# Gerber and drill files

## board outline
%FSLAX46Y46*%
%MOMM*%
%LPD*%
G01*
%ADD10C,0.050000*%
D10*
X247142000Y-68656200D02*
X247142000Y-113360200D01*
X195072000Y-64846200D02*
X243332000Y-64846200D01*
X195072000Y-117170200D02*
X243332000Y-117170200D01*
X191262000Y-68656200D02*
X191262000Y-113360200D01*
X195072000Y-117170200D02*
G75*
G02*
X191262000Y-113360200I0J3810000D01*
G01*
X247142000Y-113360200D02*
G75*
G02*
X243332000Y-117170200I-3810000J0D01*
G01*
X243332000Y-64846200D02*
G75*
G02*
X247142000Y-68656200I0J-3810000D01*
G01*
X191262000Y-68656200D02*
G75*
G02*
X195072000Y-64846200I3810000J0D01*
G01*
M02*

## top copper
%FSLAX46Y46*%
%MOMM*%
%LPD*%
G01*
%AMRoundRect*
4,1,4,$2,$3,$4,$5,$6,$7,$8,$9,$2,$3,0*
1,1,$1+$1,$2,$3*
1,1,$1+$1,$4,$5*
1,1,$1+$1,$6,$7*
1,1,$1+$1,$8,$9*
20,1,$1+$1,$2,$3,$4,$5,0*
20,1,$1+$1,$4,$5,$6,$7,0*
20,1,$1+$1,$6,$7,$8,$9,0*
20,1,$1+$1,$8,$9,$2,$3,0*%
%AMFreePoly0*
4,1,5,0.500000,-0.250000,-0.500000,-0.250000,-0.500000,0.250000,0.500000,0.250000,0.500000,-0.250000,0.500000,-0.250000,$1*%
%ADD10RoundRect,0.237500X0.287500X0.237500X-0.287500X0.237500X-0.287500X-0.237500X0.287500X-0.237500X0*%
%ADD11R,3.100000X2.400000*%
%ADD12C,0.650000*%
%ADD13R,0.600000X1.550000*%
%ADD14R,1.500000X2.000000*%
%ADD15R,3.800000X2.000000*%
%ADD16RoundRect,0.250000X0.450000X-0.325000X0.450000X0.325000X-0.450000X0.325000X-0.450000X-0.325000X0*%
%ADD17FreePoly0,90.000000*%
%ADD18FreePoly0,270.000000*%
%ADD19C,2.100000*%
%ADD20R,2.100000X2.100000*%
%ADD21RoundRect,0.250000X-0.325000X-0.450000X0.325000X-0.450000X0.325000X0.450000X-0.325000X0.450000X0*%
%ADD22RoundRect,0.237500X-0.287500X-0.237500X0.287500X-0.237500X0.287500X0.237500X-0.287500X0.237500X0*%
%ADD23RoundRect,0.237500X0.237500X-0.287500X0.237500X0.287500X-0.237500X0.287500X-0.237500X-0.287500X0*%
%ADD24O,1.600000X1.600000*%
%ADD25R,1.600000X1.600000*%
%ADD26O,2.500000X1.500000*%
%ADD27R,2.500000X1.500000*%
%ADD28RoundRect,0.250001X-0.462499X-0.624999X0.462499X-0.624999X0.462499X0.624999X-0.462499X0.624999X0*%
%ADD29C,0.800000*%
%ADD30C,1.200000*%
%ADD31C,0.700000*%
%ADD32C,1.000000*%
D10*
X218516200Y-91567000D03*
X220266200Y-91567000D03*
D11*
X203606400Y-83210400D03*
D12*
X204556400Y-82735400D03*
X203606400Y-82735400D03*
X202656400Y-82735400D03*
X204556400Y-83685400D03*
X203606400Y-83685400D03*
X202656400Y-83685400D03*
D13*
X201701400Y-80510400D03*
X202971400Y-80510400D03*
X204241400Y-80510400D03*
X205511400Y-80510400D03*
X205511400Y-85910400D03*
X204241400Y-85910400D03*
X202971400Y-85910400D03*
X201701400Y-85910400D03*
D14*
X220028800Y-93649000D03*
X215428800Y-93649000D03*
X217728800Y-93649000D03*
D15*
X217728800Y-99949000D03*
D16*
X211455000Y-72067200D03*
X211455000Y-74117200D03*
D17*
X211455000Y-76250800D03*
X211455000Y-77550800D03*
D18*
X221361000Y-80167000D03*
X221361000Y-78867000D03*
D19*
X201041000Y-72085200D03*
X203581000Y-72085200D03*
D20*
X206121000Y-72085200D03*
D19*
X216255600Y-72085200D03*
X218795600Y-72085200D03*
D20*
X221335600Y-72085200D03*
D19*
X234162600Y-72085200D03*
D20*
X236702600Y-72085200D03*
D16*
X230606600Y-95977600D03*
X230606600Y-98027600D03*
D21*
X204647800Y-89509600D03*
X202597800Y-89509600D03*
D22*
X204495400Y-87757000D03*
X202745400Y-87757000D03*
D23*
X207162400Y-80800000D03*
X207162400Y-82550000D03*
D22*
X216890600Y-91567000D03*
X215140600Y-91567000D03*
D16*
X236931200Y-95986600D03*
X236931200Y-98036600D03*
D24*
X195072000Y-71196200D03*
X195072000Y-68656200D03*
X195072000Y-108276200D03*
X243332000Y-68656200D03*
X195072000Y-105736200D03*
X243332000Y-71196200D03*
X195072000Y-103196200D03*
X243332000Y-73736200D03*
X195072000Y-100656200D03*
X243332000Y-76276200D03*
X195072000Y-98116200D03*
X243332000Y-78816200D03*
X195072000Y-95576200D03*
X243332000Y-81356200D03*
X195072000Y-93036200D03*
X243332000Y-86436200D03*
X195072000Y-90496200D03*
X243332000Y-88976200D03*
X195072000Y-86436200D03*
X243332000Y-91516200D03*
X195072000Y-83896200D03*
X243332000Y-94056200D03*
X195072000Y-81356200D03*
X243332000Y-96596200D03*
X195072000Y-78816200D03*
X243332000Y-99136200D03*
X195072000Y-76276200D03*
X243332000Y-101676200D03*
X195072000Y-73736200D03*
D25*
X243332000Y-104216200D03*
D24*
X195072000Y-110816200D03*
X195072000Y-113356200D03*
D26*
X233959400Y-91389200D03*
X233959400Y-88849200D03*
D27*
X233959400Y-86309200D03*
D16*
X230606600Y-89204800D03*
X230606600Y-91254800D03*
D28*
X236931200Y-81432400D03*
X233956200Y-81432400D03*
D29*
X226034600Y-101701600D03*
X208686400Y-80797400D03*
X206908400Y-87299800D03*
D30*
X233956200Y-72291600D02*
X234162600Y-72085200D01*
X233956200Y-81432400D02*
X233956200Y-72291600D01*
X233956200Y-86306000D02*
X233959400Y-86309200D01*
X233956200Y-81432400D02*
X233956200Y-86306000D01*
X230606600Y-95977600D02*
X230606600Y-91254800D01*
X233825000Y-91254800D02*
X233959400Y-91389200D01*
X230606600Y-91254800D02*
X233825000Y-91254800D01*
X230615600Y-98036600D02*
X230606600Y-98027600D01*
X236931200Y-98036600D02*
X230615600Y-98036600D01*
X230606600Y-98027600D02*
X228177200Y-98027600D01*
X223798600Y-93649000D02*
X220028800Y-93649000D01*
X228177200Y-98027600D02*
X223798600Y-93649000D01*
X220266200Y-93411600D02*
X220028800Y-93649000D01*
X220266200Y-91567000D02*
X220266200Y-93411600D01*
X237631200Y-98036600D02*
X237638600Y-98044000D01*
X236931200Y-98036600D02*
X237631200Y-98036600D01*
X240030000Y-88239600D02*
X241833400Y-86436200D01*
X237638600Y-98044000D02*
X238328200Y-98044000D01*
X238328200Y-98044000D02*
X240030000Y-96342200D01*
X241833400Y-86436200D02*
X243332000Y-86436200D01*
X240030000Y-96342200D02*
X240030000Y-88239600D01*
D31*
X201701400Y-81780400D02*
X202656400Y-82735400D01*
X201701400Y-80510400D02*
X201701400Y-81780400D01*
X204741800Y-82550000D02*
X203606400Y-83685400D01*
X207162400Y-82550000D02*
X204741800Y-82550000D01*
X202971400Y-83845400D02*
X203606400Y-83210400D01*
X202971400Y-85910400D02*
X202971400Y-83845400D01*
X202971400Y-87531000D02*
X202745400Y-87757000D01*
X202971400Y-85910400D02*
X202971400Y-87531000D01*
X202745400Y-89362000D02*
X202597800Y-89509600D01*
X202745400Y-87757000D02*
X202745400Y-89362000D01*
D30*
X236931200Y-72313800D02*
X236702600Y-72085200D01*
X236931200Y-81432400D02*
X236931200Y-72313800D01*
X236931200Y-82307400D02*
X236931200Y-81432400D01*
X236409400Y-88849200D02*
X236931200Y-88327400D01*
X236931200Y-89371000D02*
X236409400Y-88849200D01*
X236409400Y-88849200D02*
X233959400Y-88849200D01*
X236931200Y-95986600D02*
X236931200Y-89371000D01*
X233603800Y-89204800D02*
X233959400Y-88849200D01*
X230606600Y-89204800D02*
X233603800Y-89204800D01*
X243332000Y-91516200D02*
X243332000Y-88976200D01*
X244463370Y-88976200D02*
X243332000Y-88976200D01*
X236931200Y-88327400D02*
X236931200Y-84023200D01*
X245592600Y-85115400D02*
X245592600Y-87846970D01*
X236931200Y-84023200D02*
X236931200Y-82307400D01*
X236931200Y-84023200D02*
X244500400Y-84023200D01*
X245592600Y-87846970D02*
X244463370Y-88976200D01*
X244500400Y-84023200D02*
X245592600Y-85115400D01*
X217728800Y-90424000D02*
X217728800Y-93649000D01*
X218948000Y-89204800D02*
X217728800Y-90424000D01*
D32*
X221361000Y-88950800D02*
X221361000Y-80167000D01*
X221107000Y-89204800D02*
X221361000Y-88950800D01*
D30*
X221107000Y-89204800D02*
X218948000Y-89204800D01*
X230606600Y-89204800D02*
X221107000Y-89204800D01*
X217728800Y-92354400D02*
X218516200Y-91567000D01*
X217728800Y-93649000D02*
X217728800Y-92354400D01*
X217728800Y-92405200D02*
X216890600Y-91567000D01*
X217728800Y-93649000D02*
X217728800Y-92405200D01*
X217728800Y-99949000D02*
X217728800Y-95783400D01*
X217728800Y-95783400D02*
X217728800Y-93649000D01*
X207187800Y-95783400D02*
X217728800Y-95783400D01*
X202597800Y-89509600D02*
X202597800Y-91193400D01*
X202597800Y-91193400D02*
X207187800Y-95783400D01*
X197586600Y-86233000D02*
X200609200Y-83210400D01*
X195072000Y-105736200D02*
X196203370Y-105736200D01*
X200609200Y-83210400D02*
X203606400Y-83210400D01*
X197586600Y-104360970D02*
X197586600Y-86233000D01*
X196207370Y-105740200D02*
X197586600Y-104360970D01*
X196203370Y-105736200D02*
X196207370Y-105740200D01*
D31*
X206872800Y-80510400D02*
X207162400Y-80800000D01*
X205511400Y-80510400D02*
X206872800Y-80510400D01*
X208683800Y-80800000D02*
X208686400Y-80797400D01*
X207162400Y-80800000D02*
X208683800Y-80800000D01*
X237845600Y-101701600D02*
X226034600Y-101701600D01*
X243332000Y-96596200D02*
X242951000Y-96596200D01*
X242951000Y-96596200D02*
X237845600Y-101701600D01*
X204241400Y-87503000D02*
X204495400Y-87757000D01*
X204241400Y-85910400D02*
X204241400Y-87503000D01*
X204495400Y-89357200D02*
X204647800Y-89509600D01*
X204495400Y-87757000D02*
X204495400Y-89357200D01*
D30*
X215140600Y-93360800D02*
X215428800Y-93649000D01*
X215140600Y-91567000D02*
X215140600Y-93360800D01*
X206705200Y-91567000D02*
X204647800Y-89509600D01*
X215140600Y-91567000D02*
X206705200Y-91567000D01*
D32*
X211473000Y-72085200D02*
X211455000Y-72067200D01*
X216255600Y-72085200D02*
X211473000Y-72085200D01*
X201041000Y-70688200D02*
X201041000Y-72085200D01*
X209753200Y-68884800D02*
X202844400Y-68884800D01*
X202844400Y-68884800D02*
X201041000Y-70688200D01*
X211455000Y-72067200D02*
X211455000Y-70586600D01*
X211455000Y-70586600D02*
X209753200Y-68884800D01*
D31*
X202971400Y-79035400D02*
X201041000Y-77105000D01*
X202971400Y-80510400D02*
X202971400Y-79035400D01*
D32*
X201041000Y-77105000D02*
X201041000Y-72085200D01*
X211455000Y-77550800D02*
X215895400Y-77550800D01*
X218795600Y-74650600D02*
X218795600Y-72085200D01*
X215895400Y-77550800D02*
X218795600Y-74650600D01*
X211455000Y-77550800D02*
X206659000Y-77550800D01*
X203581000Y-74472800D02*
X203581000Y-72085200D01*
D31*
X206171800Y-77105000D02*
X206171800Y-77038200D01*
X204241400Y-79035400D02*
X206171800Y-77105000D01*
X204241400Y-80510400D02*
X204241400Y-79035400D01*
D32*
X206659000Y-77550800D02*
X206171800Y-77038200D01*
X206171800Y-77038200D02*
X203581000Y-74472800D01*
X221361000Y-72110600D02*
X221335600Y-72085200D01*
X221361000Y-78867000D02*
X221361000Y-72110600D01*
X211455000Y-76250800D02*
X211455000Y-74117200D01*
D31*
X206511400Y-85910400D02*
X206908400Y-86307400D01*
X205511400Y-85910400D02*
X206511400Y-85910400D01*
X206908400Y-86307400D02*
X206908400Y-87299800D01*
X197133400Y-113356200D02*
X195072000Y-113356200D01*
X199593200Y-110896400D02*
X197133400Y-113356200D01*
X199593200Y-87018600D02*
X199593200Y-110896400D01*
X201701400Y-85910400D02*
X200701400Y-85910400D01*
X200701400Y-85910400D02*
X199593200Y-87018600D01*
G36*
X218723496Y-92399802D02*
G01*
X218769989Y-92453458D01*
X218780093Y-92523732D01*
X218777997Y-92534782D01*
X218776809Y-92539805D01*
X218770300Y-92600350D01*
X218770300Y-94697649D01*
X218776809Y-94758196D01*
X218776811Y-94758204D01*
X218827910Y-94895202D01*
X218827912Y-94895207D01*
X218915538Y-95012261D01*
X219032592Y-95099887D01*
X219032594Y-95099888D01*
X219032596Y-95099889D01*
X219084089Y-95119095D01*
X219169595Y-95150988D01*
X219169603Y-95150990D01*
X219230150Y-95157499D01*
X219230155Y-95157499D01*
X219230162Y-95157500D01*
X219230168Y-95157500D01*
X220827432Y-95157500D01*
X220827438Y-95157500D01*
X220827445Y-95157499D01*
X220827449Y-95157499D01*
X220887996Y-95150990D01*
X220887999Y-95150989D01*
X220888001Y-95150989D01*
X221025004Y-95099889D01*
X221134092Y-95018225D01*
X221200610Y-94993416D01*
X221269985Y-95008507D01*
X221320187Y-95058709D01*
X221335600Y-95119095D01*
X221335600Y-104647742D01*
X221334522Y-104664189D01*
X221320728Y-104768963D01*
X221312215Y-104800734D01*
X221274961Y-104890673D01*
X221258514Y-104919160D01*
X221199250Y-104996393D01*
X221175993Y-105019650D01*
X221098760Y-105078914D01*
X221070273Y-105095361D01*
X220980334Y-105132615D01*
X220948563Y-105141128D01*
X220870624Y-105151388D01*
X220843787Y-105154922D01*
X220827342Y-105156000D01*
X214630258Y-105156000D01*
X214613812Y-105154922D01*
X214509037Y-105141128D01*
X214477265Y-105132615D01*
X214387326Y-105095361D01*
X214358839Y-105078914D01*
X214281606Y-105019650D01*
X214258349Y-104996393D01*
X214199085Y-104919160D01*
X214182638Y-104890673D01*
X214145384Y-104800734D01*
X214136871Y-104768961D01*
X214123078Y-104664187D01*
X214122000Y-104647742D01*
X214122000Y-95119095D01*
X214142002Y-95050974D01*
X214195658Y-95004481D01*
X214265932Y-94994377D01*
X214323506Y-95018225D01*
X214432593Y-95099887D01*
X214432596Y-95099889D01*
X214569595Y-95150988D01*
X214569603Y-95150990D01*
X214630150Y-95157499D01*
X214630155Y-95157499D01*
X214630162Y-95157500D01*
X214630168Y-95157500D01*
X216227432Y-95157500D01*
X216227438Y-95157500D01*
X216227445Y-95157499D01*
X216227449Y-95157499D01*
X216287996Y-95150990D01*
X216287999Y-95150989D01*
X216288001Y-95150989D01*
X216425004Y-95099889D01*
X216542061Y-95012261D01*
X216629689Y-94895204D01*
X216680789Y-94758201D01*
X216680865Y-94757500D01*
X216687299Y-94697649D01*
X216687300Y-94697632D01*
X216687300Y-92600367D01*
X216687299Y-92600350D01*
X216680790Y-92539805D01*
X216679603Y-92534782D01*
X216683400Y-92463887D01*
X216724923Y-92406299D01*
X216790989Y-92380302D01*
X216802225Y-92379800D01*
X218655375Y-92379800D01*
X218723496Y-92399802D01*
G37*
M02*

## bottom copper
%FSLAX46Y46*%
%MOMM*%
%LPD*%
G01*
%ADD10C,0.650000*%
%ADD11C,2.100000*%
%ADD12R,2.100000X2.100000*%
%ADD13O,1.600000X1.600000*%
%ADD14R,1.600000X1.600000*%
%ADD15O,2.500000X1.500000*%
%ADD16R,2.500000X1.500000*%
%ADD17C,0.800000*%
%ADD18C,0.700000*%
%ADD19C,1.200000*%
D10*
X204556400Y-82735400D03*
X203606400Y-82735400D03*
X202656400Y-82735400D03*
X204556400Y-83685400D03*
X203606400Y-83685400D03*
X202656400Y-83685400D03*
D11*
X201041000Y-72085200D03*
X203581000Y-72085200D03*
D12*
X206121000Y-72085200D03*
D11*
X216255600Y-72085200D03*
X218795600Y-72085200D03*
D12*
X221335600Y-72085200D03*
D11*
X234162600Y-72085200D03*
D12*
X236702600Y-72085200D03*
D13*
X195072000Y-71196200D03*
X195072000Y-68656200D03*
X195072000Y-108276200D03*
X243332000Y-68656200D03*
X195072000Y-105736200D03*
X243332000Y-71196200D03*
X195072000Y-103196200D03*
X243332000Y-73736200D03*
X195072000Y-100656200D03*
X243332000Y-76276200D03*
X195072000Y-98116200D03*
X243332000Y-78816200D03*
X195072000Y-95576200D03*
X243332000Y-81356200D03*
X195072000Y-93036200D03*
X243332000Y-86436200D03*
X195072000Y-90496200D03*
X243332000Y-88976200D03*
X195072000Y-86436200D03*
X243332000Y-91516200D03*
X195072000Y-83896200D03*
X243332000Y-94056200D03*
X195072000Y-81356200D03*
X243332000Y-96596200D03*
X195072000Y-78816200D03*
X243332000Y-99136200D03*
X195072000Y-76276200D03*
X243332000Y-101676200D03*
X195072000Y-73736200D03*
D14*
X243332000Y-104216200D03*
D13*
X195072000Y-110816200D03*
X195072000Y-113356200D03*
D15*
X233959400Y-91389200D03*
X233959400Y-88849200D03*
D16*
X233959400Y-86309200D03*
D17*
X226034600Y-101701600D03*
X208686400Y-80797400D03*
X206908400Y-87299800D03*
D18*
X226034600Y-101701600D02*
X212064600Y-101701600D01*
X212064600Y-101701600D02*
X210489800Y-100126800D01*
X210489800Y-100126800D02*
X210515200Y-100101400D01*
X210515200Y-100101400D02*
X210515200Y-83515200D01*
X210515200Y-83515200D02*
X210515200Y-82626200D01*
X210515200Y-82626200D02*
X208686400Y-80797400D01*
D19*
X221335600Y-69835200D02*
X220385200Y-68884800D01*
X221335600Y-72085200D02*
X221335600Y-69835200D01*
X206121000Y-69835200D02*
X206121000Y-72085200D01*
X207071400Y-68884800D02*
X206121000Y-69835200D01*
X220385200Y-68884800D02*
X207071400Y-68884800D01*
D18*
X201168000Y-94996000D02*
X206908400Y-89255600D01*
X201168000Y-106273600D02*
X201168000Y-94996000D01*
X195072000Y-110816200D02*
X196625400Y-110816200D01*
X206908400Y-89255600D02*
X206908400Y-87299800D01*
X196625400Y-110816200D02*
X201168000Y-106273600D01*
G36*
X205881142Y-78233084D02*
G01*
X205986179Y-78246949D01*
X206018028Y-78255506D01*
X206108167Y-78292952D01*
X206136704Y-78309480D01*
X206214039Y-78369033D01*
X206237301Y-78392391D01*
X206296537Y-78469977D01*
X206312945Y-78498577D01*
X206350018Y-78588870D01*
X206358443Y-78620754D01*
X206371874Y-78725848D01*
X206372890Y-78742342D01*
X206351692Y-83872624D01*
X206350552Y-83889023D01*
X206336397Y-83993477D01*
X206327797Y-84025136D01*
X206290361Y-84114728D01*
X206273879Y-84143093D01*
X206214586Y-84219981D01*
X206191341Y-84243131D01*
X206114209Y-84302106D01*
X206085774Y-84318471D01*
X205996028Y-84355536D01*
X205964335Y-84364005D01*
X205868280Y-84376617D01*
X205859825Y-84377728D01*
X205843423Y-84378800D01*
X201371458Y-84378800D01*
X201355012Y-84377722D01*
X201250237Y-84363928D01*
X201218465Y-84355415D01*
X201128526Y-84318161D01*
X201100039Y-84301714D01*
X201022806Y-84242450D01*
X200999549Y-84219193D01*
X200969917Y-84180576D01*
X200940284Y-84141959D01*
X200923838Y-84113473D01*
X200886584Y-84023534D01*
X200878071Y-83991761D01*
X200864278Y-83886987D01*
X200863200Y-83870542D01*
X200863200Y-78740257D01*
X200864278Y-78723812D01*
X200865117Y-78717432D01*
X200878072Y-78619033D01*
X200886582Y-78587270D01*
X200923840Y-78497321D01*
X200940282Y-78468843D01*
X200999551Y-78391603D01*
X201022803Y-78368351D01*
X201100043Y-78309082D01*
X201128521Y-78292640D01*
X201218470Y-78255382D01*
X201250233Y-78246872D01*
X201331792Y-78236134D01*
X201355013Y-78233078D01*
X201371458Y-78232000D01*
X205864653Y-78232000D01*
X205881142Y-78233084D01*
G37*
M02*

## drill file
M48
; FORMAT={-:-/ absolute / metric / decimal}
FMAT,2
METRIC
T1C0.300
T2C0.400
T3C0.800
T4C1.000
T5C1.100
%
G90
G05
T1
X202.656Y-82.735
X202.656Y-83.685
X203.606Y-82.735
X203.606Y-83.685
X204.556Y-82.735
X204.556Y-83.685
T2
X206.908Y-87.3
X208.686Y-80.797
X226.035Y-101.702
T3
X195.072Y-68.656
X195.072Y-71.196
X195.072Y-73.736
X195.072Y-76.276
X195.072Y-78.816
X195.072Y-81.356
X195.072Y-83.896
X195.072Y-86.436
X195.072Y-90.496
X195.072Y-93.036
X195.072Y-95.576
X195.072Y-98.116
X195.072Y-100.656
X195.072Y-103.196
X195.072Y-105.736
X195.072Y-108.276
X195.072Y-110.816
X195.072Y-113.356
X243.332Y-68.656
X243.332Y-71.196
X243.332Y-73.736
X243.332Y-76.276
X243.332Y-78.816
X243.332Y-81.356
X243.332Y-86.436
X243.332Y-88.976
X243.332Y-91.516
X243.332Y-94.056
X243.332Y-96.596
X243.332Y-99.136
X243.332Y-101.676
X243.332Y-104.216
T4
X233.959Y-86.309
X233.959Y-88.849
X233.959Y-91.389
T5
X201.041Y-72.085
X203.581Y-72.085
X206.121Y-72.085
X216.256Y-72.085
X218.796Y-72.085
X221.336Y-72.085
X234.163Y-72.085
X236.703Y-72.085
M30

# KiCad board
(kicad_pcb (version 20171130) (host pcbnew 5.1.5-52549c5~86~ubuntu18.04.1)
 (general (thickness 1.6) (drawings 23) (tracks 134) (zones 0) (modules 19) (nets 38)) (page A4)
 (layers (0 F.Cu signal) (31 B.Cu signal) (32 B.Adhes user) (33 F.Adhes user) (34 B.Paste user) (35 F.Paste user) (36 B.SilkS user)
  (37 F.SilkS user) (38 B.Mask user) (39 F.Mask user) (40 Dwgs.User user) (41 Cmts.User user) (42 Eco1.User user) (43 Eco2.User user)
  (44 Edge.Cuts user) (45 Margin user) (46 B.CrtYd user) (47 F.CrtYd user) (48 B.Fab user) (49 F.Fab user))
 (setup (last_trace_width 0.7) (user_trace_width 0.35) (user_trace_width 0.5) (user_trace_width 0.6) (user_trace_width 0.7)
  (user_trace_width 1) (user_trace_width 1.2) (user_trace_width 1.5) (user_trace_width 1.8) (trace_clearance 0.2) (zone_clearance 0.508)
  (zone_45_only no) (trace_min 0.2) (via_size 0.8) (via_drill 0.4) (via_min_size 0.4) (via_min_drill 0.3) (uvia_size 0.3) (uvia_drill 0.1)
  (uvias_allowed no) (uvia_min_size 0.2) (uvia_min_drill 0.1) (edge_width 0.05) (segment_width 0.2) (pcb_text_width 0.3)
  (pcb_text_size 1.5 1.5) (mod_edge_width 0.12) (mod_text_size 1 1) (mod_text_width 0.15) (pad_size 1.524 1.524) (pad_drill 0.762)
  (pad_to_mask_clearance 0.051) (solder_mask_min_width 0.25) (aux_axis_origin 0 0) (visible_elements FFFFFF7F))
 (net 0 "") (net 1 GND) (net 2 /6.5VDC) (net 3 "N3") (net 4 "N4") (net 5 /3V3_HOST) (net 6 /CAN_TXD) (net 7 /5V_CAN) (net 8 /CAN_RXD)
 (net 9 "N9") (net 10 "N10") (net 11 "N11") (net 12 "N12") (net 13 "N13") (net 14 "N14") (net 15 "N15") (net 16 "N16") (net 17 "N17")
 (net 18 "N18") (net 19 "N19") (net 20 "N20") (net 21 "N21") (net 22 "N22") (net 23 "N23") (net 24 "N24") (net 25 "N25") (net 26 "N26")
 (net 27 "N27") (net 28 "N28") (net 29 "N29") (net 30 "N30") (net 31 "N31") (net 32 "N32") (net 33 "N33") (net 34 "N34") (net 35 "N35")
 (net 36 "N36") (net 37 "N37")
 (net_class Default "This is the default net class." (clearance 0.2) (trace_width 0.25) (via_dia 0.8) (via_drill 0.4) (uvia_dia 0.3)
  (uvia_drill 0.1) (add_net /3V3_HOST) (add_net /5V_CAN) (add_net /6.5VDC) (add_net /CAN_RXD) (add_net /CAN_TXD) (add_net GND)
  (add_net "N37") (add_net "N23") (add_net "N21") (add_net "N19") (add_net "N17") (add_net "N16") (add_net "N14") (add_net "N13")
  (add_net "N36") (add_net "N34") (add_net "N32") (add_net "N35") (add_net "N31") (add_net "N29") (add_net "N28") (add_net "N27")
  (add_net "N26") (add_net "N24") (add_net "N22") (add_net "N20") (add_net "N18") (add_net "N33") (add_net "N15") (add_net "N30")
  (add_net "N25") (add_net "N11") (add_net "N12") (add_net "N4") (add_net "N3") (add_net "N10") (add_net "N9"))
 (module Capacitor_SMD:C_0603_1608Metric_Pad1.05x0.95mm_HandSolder (layer F.Cu) (at 219.3912 91.567 180)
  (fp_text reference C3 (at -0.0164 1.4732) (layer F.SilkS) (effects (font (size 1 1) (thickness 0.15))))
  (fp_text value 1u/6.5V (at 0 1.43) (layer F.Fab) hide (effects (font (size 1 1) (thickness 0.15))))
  (pad 2 smd roundrect (at 0.875 0 180) (size 1.05 0.95) (layers F.Cu F.Paste F.Mask) (roundrect_rratio 0.25) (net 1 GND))
  (pad 1 smd roundrect (at -0.875 0 180) (size 1.05 0.95) (layers F.Cu F.Paste F.Mask) (roundrect_rratio 0.25) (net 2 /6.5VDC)))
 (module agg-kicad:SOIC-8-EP (layer F.Cu) (at 203.6064 83.2104 90)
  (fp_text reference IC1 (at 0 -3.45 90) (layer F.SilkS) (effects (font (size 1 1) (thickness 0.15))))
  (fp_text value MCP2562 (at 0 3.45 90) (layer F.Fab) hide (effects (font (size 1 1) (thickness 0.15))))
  (pad EP smd rect (at 0 0 90) (size 2.4 3.1) (layers F.Cu F.Paste F.Mask) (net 1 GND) (solder_mask_margin 0.001)
   (solder_paste_margin 0.001))
  (pad EP thru_hole circle (at 0.475 0.95 90) (size 0.65 0.65) (drill 0.3) (layers *.Cu) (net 1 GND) (zone_connect 2))
  (pad EP thru_hole circle (at 0.475 0 90) (size 0.65 0.65) (drill 0.3) (layers *.Cu) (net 1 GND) (zone_connect 2))
  (pad EP thru_hole circle (at 0.475 -0.95 90) (size 0.65 0.65) (drill 0.3) (layers *.Cu) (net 1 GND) (zone_connect 2))
  (pad EP thru_hole circle (at -0.475 0.95 90) (size 0.65 0.65) (drill 0.3) (layers *.Cu) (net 1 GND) (zone_connect 2))
  (pad EP thru_hole circle (at -0.475 0 90) (size 0.65 0.65) (drill 0.3) (layers *.Cu) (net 1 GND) (zone_connect 2))
  (pad EP thru_hole circle (at -0.475 -0.95 90) (size 0.65 0.65) (drill 0.3) (layers *.Cu) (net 1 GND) (zone_connect 2))
  (pad 8 smd rect (at 2.7 -1.905 90) (size 1.55 0.6) (layers F.Cu F.Paste F.Mask) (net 1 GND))
  (pad 7 smd rect (at 2.7 -0.635 90) (size 1.55 0.6) (layers F.Cu F.Paste F.Mask) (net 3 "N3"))
  (pad 6 smd rect (at 2.7 0.635 90) (size 1.55 0.6) (layers F.Cu F.Paste F.Mask) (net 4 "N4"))
  (pad 5 smd rect (at 2.7 1.905 90) (size 1.55 0.6) (layers F.Cu F.Paste F.Mask) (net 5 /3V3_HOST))
  (pad 4 smd rect (at -2.7 1.905 90) (size 1.55 0.6) (layers F.Cu F.Paste F.Mask) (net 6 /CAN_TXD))
  (pad 3 smd rect (at -2.7 0.635 90) (size 1.55 0.6) (layers F.Cu F.Paste F.Mask) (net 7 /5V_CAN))
  (pad 2 smd rect (at -2.7 -0.635 90) (size 1.55 0.6) (layers F.Cu F.Paste F.Mask) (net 1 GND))
  (pad 1 smd rect (at -2.7 -1.905 90) (size 1.55 0.6) (layers F.Cu F.Paste F.Mask) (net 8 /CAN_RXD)))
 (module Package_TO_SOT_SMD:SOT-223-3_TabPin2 (layer F.Cu) (at 217.7288 96.799 270)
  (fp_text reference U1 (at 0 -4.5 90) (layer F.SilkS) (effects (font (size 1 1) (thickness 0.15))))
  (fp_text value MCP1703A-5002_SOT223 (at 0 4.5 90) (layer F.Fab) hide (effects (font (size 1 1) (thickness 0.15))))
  (pad 1 smd rect (at -3.15 -2.3 270) (size 2 1.5) (layers F.Cu F.Paste F.Mask) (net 2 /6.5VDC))
  (pad 3 smd rect (at -3.15 2.3 270) (size 2 1.5) (layers F.Cu F.Paste F.Mask) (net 7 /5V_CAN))
  (pad 2 smd rect (at -3.15 0 270) (size 2 1.5) (layers F.Cu F.Paste F.Mask) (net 1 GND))
  (pad 2 smd rect (at 3.15 0 270) (size 2 3.8) (layers F.Cu F.Paste F.Mask) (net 1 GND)))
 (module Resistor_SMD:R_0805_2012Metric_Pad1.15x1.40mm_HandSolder (layer F.Cu) (at 211.455 73.0922 90)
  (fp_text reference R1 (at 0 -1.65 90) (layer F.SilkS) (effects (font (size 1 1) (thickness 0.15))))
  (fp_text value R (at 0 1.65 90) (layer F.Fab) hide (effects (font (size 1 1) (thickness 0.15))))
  (pad 2 smd roundrect (at 1.025 0 90) (size 1.15 1.4) (layers F.Cu F.Paste F.Mask) (roundrect_rratio 0.217391) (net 3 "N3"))
  (pad 1 smd roundrect (at -1.025 0 90) (size 1.15 1.4) (layers F.Cu F.Paste F.Mask) (roundrect_rratio 0.217391) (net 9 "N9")))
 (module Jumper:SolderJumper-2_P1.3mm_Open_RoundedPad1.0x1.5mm (layer F.Cu) (at 211.455 76.9008 90)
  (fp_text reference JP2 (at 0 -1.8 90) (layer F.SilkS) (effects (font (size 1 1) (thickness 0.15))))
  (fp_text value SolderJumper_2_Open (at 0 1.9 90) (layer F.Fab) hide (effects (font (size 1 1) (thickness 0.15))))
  (pad 2 smd custom (at 0.65 0 90) (size 1 0.5) (layers F.Cu F.Mask) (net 9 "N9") (zone_connect 2)
   (options (clearance outline) (anchor rect)) (primitives))
  (pad 1 smd custom (at -0.65 0 90) (size 1 0.5) (layers F.Cu F.Mask) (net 4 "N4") (zone_connect 2)
   (options (clearance outline) (anchor rect)) (primitives)))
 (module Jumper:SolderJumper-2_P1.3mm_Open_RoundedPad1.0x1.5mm (layer F.Cu) (at 221.361 79.517 270)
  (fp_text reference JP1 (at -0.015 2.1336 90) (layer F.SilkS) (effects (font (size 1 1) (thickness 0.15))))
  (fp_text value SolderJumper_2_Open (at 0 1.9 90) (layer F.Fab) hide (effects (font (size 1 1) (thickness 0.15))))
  (pad 2 smd custom (at 0.65 0 270) (size 1 0.5) (layers F.Cu F.Mask) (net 1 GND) (zone_connect 2)
   (options (clearance outline) (anchor rect)) (primitives))
  (pad 1 smd custom (at -0.65 0 270) (size 1 0.5) (layers F.Cu F.Mask) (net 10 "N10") (zone_connect 2)
   (options (clearance outline) (anchor rect)) (primitives)))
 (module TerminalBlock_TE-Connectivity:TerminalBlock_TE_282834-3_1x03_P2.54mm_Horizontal (layer F.Cu) (at 206.121 72.0852 180)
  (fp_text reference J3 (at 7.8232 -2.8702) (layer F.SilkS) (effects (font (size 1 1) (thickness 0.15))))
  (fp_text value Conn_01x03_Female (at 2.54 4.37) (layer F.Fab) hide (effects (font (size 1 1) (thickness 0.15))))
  (pad 3 thru_hole circle (at 5.08 0 180) (size 2.1 2.1) (drill 1.1) (layers *.Cu *.Mask) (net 3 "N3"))
  (pad 2 thru_hole circle (at 2.54 0 180) (size 2.1 2.1) (drill 1.1) (layers *.Cu *.Mask) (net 4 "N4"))
  (pad 1 thru_hole rect (at 0 0 180) (size 2.1 2.1) (drill 1.1) (layers *.Cu *.Mask) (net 10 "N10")))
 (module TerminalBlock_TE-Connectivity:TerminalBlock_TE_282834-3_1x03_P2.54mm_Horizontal (layer F.Cu) (at 221.3356 72.0852 180)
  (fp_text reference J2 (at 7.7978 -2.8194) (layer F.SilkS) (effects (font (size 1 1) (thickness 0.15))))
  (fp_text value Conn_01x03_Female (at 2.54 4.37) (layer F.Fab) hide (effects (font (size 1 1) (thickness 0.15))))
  (pad 3 thru_hole circle (at 5.08 0 180) (size 2.1 2.1) (drill 1.1) (layers *.Cu *.Mask) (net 3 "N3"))
  (pad 2 thru_hole circle (at 2.54 0 180) (size 2.1 2.1) (drill 1.1) (layers *.Cu *.Mask) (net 4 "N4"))
  (pad 1 thru_hole rect (at 0 0 180) (size 2.1 2.1) (drill 1.1) (layers *.Cu *.Mask) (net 10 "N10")))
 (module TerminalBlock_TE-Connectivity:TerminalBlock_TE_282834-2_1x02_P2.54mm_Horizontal (layer F.Cu) (at 236.7026 72.0852 180)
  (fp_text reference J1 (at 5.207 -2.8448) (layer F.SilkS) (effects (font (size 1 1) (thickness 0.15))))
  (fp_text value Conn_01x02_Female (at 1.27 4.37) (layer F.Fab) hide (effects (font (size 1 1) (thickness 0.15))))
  (pad 2 thru_hole circle (at 2.54 0 180) (size 2.1 2.1) (drill 1.1) (layers *.Cu *.Mask) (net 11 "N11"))
  (pad 1 thru_hole rect (at 0 0 180) (size 2.1 2.1) (drill 1.1) (layers *.Cu *.Mask) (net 1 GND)))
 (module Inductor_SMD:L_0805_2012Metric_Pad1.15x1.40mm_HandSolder (layer F.Cu) (at 230.6066 97.0026 90)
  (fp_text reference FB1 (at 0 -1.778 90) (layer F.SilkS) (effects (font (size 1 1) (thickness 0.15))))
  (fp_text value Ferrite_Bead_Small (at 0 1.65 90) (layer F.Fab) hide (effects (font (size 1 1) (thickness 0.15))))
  (pad 2 smd roundrect (at 1.025 0 90) (size 1.15 1.4) (layers F.Cu F.Paste F.Mask) (roundrect_rratio 0.217391) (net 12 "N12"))
  (pad 1 smd roundrect (at -1.025 0 90) (size 1.15 1.4) (layers F.Cu F.Paste F.Mask) (roundrect_rratio 0.217391) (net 2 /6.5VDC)))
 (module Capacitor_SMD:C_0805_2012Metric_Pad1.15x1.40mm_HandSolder (layer F.Cu) (at 203.6228 89.5096)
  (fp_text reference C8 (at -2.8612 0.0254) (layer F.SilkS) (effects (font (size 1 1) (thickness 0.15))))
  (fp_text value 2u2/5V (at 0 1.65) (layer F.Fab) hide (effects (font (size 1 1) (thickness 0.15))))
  (pad 2 smd roundrect (at 1.025 0) (size 1.15 1.4) (layers F.Cu F.Paste F.Mask) (roundrect_rratio 0.217391) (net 7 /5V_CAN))
  (pad 1 smd roundrect (at -1.025 0) (size 1.15 1.4) (layers F.Cu F.Paste F.Mask) (roundrect_rratio 0.217391) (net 1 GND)))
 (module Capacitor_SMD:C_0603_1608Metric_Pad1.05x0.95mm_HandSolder (layer F.Cu) (at 203.6204 87.757)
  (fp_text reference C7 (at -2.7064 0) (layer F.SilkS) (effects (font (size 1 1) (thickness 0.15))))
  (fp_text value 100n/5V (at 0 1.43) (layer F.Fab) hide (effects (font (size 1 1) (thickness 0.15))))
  (pad 2 smd roundrect (at 0.875 0) (size 1.05 0.95) (layers F.Cu F.Paste F.Mask) (roundrect_rratio 0.25) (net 7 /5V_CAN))
  (pad 1 smd roundrect (at -0.875 0) (size 1.05 0.95) (layers F.Cu F.Paste F.Mask) (roundrect_rratio 0.25) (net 1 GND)))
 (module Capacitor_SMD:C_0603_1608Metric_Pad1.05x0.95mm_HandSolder (layer F.Cu) (at 207.1624 81.675 90)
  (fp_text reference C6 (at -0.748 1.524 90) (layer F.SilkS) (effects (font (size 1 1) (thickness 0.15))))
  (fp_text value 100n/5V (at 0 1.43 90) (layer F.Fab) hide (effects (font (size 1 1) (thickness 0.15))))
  (pad 2 smd roundrect (at 0.875 0 90) (size 1.05 0.95) (layers F.Cu F.Paste F.Mask) (roundrect_rratio 0.25) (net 5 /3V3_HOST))
  (pad 1 smd roundrect (at -0.875 0 90) (size 1.05 0.95) (layers F.Cu F.Paste F.Mask) (roundrect_rratio 0.25) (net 1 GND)))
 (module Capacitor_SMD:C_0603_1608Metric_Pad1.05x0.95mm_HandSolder (layer F.Cu) (at 216.0156 91.567)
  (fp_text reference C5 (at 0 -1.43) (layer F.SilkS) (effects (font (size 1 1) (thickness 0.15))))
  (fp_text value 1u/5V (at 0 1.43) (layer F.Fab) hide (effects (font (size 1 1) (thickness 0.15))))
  (pad 2 smd roundrect (at 0.875 0) (size 1.05 0.95) (layers F.Cu F.Paste F.Mask) (roundrect_rratio 0.25) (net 1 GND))
  (pad 1 smd roundrect (at -0.875 0) (size 1.05 0.95) (layers F.Cu F.Paste F.Mask) (roundrect_rratio 0.25) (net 7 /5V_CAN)))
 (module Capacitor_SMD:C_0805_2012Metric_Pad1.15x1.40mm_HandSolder (layer F.Cu) (at 236.9312 97.0116 90)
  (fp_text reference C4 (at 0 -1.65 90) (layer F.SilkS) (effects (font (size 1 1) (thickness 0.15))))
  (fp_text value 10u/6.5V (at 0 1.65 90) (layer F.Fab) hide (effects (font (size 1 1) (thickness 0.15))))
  (pad 2 smd roundrect (at 1.025 0 90) (size 1.15 1.4) (layers F.Cu F.Paste F.Mask) (roundrect_rratio 0.217391) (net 1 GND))
  (pad 1 smd roundrect (at -1.025 0 90) (size 1.15 1.4) (layers F.Cu F.Paste F.Mask) (roundrect_rratio 0.217391) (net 2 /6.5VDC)))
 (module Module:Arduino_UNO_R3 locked (layer B.Cu) (at 243.332 104.2162 90)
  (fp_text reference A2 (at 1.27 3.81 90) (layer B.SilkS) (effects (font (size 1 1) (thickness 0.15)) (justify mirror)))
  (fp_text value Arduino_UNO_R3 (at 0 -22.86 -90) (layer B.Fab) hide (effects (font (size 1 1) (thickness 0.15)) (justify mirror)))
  (pad 16 thru_hole oval (at 33.02 -48.26) (size 1.6 1.6) (drill 0.8) (layers *.Cu *.Mask) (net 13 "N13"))
  (pad 15 thru_hole oval (at 35.56 -48.26) (size 1.6 1.6) (drill 0.8) (layers *.Cu *.Mask) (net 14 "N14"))
  (pad 30 thru_hole oval (at -4.06 -48.26) (size 1.6 1.6) (drill 0.8) (layers *.Cu *.Mask) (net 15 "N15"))
  (pad 14 thru_hole oval (at 35.56 0) (size 1.6 1.6) (drill 0.8) (layers *.Cu *.Mask) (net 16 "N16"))
  (pad 29 thru_hole oval (at -1.52 -48.26) (size 1.6 1.6) (drill 0.8) (layers *.Cu *.Mask) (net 1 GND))
  (pad 13 thru_hole oval (at 33.02 0) (size 1.6 1.6) (drill 0.8) (layers *.Cu *.Mask) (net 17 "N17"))
  (pad 28 thru_hole oval (at 1.02 -48.26) (size 1.6 1.6) (drill 0.8) (layers *.Cu *.Mask) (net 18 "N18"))
  (pad 12 thru_hole oval (at 30.48 0) (size 1.6 1.6) (drill 0.8) (layers *.Cu *.Mask) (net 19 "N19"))
  (pad 27 thru_hole oval (at 3.56 -48.26) (size 1.6 1.6) (drill 0.8) (layers *.Cu *.Mask) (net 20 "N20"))
  (pad 11 thru_hole oval (at 27.94 0) (size 1.6 1.6) (drill 0.8) (layers *.Cu *.Mask) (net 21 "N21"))
  (pad 26 thru_hole oval (at 6.1 -48.26) (size 1.6 1.6) (drill 0.8) (layers *.Cu *.Mask) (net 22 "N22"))
  (pad 10 thru_hole oval (at 25.4 0) (size 1.6 1.6) (drill 0.8) (layers *.Cu *.Mask) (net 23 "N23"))
  (pad 25 thru_hole oval (at 8.64 -48.26) (size 1.6 1.6) (drill 0.8) (layers *.Cu *.Mask) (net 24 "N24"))
  (pad 9 thru_hole oval (at 22.86 0) (size 1.6 1.6) (drill 0.8) (layers *.Cu *.Mask) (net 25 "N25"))
  (pad 24 thru_hole oval (at 11.18 -48.26) (size 1.6 1.6) (drill 0.8) (layers *.Cu *.Mask) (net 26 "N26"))
  (pad 8 thru_hole oval (at 17.78 0) (size 1.6 1.6) (drill 0.8) (layers *.Cu *.Mask) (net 2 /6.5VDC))
  (pad 23 thru_hole oval (at 13.72 -48.26) (size 1.6 1.6) (drill 0.8) (layers *.Cu *.Mask) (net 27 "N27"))
  (pad 7 thru_hole oval (at 15.24 0) (size 1.6 1.6) (drill 0.8) (layers *.Cu *.Mask) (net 1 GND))
  (pad 22 thru_hole oval (at 17.78 -48.26) (size 1.6 1.6) (drill 0.8) (layers *.Cu *.Mask) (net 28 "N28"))
  (pad 6 thru_hole oval (at 12.7 0) (size 1.6 1.6) (drill 0.8) (layers *.Cu *.Mask) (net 1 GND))
  (pad 21 thru_hole oval (at 20.32 -48.26) (size 1.6 1.6) (drill 0.8) (layers *.Cu *.Mask) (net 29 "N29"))
  (pad 5 thru_hole oval (at 10.16 0) (size 1.6 1.6) (drill 0.8) (layers *.Cu *.Mask) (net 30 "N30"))
  (pad 20 thru_hole oval (at 22.86 -48.26) (size 1.6 1.6) (drill 0.8) (layers *.Cu *.Mask) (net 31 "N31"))
  (pad 4 thru_hole oval (at 7.62 0) (size 1.6 1.6) (drill 0.8) (layers *.Cu *.Mask) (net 5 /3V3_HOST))
  (pad 19 thru_hole oval (at 25.4 -48.26) (size 1.6 1.6) (drill 0.8) (layers *.Cu *.Mask) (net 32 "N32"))
  (pad 3 thru_hole oval (at 5.08 0) (size 1.6 1.6) (drill 0.8) (layers *.Cu *.Mask) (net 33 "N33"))
  (pad 18 thru_hole oval (at 27.94 -48.26) (size 1.6 1.6) (drill 0.8) (layers *.Cu *.Mask) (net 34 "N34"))
  (pad 2 thru_hole oval (at 2.54 0) (size 1.6 1.6) (drill 0.8) (layers *.Cu *.Mask) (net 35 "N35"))
  (pad 17 thru_hole oval (at 30.48 -48.26) (size 1.6 1.6) (drill 0.8) (layers *.Cu *.Mask) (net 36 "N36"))
  (pad 1 thru_hole rect (at 0 0) (size 1.6 1.6) (drill 0.8) (layers *.Cu *.Mask) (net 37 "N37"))
  (pad 31 thru_hole oval (at -6.6 -48.26) (size 1.6 1.6) (drill 0.8) (layers *.Cu *.Mask) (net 6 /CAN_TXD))
  (pad 32 thru_hole oval (at -9.14 -48.26) (size 1.6 1.6) (drill 0.8) (layers *.Cu *.Mask) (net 8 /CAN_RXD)))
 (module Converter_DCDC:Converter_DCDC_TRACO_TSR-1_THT (layer F.Cu) (at 233.9594 86.3092 270)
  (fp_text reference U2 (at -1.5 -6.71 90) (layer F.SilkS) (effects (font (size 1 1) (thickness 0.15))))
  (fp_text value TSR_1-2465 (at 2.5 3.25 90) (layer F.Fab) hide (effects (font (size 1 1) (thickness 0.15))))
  (pad 3 thru_hole oval (at 5.08 0 270) (size 1.5 2.5) (drill 1) (layers *.Cu *.Mask) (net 12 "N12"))
  (pad 2 thru_hole oval (at 2.54 0 270) (size 1.5 2.5) (drill 1) (layers *.Cu *.Mask) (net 1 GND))
  (pad 1 thru_hole rect (at 0 0 270) (size 1.5 2.5) (drill 1) (layers *.Cu *.Mask) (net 11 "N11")))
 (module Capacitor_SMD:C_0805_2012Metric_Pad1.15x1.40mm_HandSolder (layer F.Cu) (at 230.6066 90.2298 90)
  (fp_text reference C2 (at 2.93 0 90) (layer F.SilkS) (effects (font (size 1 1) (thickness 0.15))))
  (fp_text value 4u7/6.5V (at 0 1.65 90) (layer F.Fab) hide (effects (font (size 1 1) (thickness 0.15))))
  (pad 2 smd roundrect (at 1.025 0 90) (size 1.15 1.4) (layers F.Cu F.Paste F.Mask) (roundrect_rratio 0.217391) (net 1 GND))
  (pad 1 smd roundrect (at -1.025 0 90) (size 1.15 1.4) (layers F.Cu F.Paste F.Mask) (roundrect_rratio 0.217391) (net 12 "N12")))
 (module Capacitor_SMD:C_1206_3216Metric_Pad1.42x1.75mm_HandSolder (layer F.Cu) (at 235.4437 81.4324)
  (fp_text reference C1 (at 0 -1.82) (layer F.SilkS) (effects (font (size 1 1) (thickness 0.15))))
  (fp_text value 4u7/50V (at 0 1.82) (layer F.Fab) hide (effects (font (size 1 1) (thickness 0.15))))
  (pad 2 smd roundrect (at 1.4875 0) (size 1.425 1.75) (layers F.Cu F.Paste F.Mask) (roundrect_rratio 0.175439) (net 1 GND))
  (pad 1 smd roundrect (at -1.4875 0) (size 1.425 1.75) (layers F.Cu F.Paste F.Mask) (roundrect_rratio 0.175439) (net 11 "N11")))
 (gr_line (start 247.142 68.6562) (end 247.142 113.3602) (layer Edge.Cuts) (width 0.05))
 (gr_line (start 195.072 64.8462) (end 243.332 64.8462) (layer Edge.Cuts) (width 0.05))
 (gr_line (start 195.072 117.1702) (end 243.332 117.1702) (layer Edge.Cuts) (width 0.05))
 (gr_line (start 191.262 68.6562) (end 191.262 113.3602) (layer Edge.Cuts) (width 0.05))
 (gr_arc (start 195.072 113.3602) (end 191.262 113.3602) (angle -90) (layer Edge.Cuts) (width 0.05))
 (gr_arc (start 243.332 113.3602) (end 243.332 117.1702) (angle -90) (layer Edge.Cuts) (width 0.05))
 (gr_arc (start 243.332 68.6562) (end 247.142 68.6562) (angle -90) (layer Edge.Cuts) (width 0.05))
 (gr_arc (start 195.072 68.6562) (end 195.072 64.8462) (angle -90) (layer Edge.Cuts) (width 0.05))
 (segment (start 233.9562 72.2916) (end 234.1626 72.0852) (width 1.2) (layer F.Cu) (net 11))
 (segment (start 233.9562 81.4324) (end 233.9562 72.2916) (width 1.2) (layer F.Cu) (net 11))
 (segment (start 233.9562 86.306) (end 233.9594 86.3092) (width 1.2) (layer F.Cu) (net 11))
 (segment (start 233.9562 81.4324) (end 233.9562 86.306) (width 1.2) (layer F.Cu) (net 11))
 (segment (start 230.6066 95.9776) (end 230.6066 91.2548) (width 1.2) (layer F.Cu) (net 12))
 (segment (start 233.825 91.2548) (end 233.9594 91.3892) (width 1.2) (layer F.Cu) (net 12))
 (segment (start 230.6066 91.2548) (end 233.825 91.2548) (width 1.2) (layer F.Cu) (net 12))
 (segment (start 230.6156 98.0366) (end 230.6066 98.0276) (width 1.2) (layer F.Cu) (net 2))
 (segment (start 236.9312 98.0366) (end 230.6156 98.0366) (width 1.2) (layer F.Cu) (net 2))
 (segment (start 230.6066 98.0276) (end 228.1772 98.0276) (width 1.2) (layer F.Cu) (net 2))
 (segment (start 223.7986 93.649) (end 220.0288 93.649) (width 1.2) (layer F.Cu) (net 2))
 (segment (start 228.1772 98.0276) (end 223.7986 93.649) (width 1.2) (layer F.Cu) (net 2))
 (segment (start 220.2662 93.4116) (end 220.0288 93.649) (width 1.2) (layer F.Cu) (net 2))
 (segment (start 220.2662 91.567) (end 220.2662 93.4116) (width 1.2) (layer F.Cu) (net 2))
 (segment (start 237.6312 98.0366) (end 237.6386 98.044) (width 1.2) (layer F.Cu) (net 2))
 (segment (start 236.9312 98.0366) (end 237.6312 98.0366) (width 1.2) (layer F.Cu) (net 2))
 (segment (start 240.03 88.2396) (end 241.8334 86.4362) (width 1.2) (layer F.Cu) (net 2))
 (segment (start 237.6386 98.044) (end 238.3282 98.044) (width 1.2) (layer F.Cu) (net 2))
 (segment (start 238.3282 98.044) (end 240.03 96.3422) (width 1.2) (layer F.Cu) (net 2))
 (segment (start 241.8334 86.4362) (end 243.332 86.4362) (width 1.2) (layer F.Cu) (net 2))
 (segment (start 240.03 96.3422) (end 240.03 88.2396) (width 1.2) (layer F.Cu) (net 2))
 (segment (start 201.7014 81.7804) (end 202.6564 82.7354) (width 0.7) (layer F.Cu) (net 1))
 (segment (start 201.7014 80.5104) (end 201.7014 81.7804) (width 0.7) (layer F.Cu) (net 1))
 (segment (start 204.7418 82.55) (end 203.6064 83.6854) (width 0.7) (layer F.Cu) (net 1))
 (segment (start 207.1624 82.55) (end 204.7418 82.55) (width 0.7) (layer F.Cu) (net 1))
 (segment (start 202.9714 83.8454) (end 203.6064 83.2104) (width 0.7) (layer F.Cu) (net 1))
 (segment (start 202.9714 85.9104) (end 202.9714 83.8454) (width 0.7) (layer F.Cu) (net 1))
 (segment (start 202.9714 87.531) (end 202.7454 87.757) (width 0.7) (layer F.Cu) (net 1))
 (segment (start 202.9714 85.9104) (end 202.9714 87.531) (width 0.7) (layer F.Cu) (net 1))
 (segment (start 202.7454 89.362) (end 202.5978 89.5096) (width 0.7) (layer F.Cu) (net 1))
 (segment (start 202.7454 87.757) (end 202.7454 89.362) (width 0.7) (layer F.Cu) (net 1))
 (segment (start 236.9312 72.3138) (end 236.7026 72.0852) (width 1.2) (layer F.Cu) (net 1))
 (segment (start 236.9312 81.4324) (end 236.9312 72.3138) (width 1.2) (layer F.Cu) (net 1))
 (segment (start 236.9312 82.3074) (end 236.9312 81.4324) (width 1.2) (layer F.Cu) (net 1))
 (segment (start 236.4094 88.8492) (end 236.9312 88.3274) (width 1.2) (layer F.Cu) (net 1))
 (segment (start 236.9312 89.371) (end 236.4094 88.8492) (width 1.2) (layer F.Cu) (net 1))
 (segment (start 236.4094 88.8492) (end 233.9594 88.8492) (width 1.2) (layer F.Cu) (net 1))
 (segment (start 236.9312 95.9866) (end 236.9312 89.371) (width 1.2) (layer F.Cu) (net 1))
 (segment (start 233.6038 89.2048) (end 233.9594 88.8492) (width 1.2) (layer F.Cu) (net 1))
 (segment (start 230.6066 89.2048) (end 233.6038 89.2048) (width 1.2) (layer F.Cu) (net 1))
 (segment (start 243.332 91.5162) (end 243.332 88.9762) (width 1.2) (layer F.Cu) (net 1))
 (segment (start 244.46337 88.9762) (end 243.332 88.9762) (width 1.2) (layer F.Cu) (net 1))
 (segment (start 236.9312 88.3274) (end 236.9312 84.0232) (width 1.2) (layer F.Cu) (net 1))
 (segment (start 245.5926 85.1154) (end 245.5926 87.84697) (width 1.2) (layer F.Cu) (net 1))
 (segment (start 236.9312 84.0232) (end 236.9312 82.3074) (width 1.2) (layer F.Cu) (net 1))
 (segment (start 236.9312 84.0232) (end 244.5004 84.0232) (width 1.2) (layer F.Cu) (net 1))
 (segment (start 245.5926 87.84697) (end 244.46337 88.9762) (width 1.2) (layer F.Cu) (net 1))
 (segment (start 244.5004 84.0232) (end 245.5926 85.1154) (width 1.2) (layer F.Cu) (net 1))
 (segment (start 217.7288 90.424) (end 217.7288 93.649) (width 1.2) (layer F.Cu) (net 1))
 (segment (start 218.948 89.2048) (end 217.7288 90.424) (width 1.2) (layer F.Cu) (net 1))
 (segment (start 221.361 88.9508) (end 221.361 80.167) (width 1) (layer F.Cu) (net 1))
 (segment (start 221.107 89.2048) (end 221.361 88.9508) (width 1) (layer F.Cu) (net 1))
 (segment (start 221.107 89.2048) (end 218.948 89.2048) (width 1.2) (layer F.Cu) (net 1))
 (segment (start 230.6066 89.2048) (end 221.107 89.2048) (width 1.2) (layer F.Cu) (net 1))
 (segment (start 217.7288 92.3544) (end 218.5162 91.567) (width 1.2) (layer F.Cu) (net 1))
 (segment (start 217.7288 93.649) (end 217.7288 92.3544) (width 1.2) (layer F.Cu) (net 1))
 (segment (start 217.7288 92.4052) (end 216.8906 91.567) (width 1.2) (layer F.Cu) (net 1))
 (segment (start 217.7288 93.649) (end 217.7288 92.4052) (width 1.2) (layer F.Cu) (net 1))
 (segment (start 217.7288 99.949) (end 217.7288 95.7834) (width 1.2) (layer F.Cu) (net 1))
 (segment (start 217.7288 95.7834) (end 217.7288 93.649) (width 1.2) (layer F.Cu) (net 1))
 (segment (start 207.1878 95.7834) (end 217.7288 95.7834) (width 1.2) (layer F.Cu) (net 1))
 (segment (start 202.5978 89.5096) (end 202.5978 91.1934) (width 1.2) (layer F.Cu) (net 1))
 (segment (start 202.5978 91.1934) (end 207.1878 95.7834) (width 1.2) (layer F.Cu) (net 1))
 (segment (start 197.5866 86.233) (end 200.6092 83.2104) (width 1.2) (layer F.Cu) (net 1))
 (segment (start 195.072 105.7362) (end 196.20337 105.7362) (width 1.2) (layer F.Cu) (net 1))
 (segment (start 200.6092 83.2104) (end 203.6064 83.2104) (width 1.2) (layer F.Cu) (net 1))
 (segment (start 197.5866 104.36097) (end 197.5866 86.233) (width 1.2) (layer F.Cu) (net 1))
 (segment (start 196.20737 105.7402) (end 197.5866 104.36097) (width 1.2) (layer F.Cu) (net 1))
 (segment (start 196.20337 105.7362) (end 196.20737 105.7402) (width 1.2) (layer F.Cu) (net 1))
 (segment (start 206.8728 80.5104) (end 207.1624 80.8) (width 0.7) (layer F.Cu) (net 5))
 (segment (start 205.5114 80.5104) (end 206.8728 80.5104) (width 0.7) (layer F.Cu) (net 5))
 (via (at 226.0346 101.7016) (size 0.8) (drill 0.4) (layers F.Cu B.Cu) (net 5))
 (segment (start 226.0346 101.7016) (end 212.0646 101.7016) (width 0.7) (layer B.Cu) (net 5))
 (segment (start 212.0646 101.7016) (end 210.4898 100.1268) (width 0.7) (layer B.Cu) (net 5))
 (segment (start 210.4898 100.1268) (end 210.5152 100.1014) (width 0.7) (layer B.Cu) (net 5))
 (segment (start 210.5152 100.1014) (end 210.5152 83.5152) (width 0.7) (layer B.Cu) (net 5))
 (segment (start 210.5152 83.5152) (end 210.5152 82.6262) (width 0.7) (layer B.Cu) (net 5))
 (segment (start 210.5152 82.6262) (end 208.6864 80.7974) (width 0.7) (layer B.Cu) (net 5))
 (via (at 208.6864 80.7974) (size 0.8) (drill 0.4) (layers F.Cu B.Cu) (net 5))
 (segment (start 208.6838 80.8) (end 208.6864 80.7974) (width 0.7) (layer F.Cu) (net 5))
 (segment (start 207.1624 80.8) (end 208.6838 80.8) (width 0.7) (layer F.Cu) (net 5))
 (segment (start 237.8456 101.7016) (end 226.0346 101.7016) (width 0.7) (layer F.Cu) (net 5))
 (segment (start 243.332 96.5962) (end 242.951 96.5962) (width 0.7) (layer F.Cu) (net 5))
 (segment (start 242.951 96.5962) (end 237.8456 101.7016) (width 0.7) (layer F.Cu) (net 5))
 (segment (start 204.2414 87.503) (end 204.4954 87.757) (width 0.7) (layer F.Cu) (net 7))
 (segment (start 204.2414 85.9104) (end 204.2414 87.503) (width 0.7) (layer F.Cu) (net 7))
 (segment (start 204.4954 89.3572) (end 204.6478 89.5096) (width 0.7) (layer F.Cu) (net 7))
 (segment (start 204.4954 87.757) (end 204.4954 89.3572) (width 0.7) (layer F.Cu) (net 7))
 (segment (start 215.1406 93.3608) (end 215.4288 93.649) (width 1.2) (layer F.Cu) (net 7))
 (segment (start 215.1406 91.567) (end 215.1406 93.3608) (width 1.2) (layer F.Cu) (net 7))
 (segment (start 206.7052 91.567) (end 204.6478 89.5096) (width 1.2) (layer F.Cu) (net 7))
 (segment (start 215.1406 91.567) (end 206.7052 91.567) (width 1.2) (layer F.Cu) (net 7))
 (segment (start 211.473 72.0852) (end 211.455 72.0672) (width 1) (layer F.Cu) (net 3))
 (segment (start 216.2556 72.0852) (end 211.473 72.0852) (width 1) (layer F.Cu) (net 3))
 (segment (start 201.041 70.6882) (end 201.041 72.0852) (width 1) (layer F.Cu) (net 3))
 (segment (start 209.7532 68.8848) (end 202.8444 68.8848) (width 1) (layer F.Cu) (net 3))
 (segment (start 202.8444 68.8848) (end 201.041 70.6882) (width 1) (layer F.Cu) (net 3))
 (segment (start 211.455 72.0672) (end 211.455 70.5866) (width 1) (layer F.Cu) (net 3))
 (segment (start 211.455 70.5866) (end 209.7532 68.8848) (width 1) (layer F.Cu) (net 3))
 (segment (start 202.9714 79.0354) (end 201.041 77.105) (width 0.7) (layer F.Cu) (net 3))
 (segment (start 202.9714 80.5104) (end 202.9714 79.0354) (width 0.7) (layer F.Cu) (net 3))
 (segment (start 201.041 77.105) (end 201.041 72.0852) (width 1) (layer F.Cu) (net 3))
 (segment (start 211.455 77.5508) (end 215.8954 77.5508) (width 1) (layer F.Cu) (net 4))
 (segment (start 218.7956 74.6506) (end 218.7956 72.0852) (width 1) (layer F.Cu) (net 4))
 (segment (start 215.8954 77.5508) (end 218.7956 74.6506) (width 1) (layer F.Cu) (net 4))
 (segment (start 211.455 77.5508) (end 206.659 77.5508) (width 1) (layer F.Cu) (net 4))
 (segment (start 203.581 74.4728) (end 203.581 72.0852) (width 1) (layer F.Cu) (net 4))
 (segment (start 206.1718 77.105) (end 206.1718 77.0382) (width 0.7) (layer F.Cu) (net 4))
 (segment (start 204.2414 79.0354) (end 206.1718 77.105) (width 0.7) (layer F.Cu) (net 4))
 (segment (start 204.2414 80.5104) (end 204.2414 79.0354) (width 0.7) (layer F.Cu) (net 4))
 (segment (start 206.659 77.5508) (end 206.1718 77.0382) (width 1) (layer F.Cu) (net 4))
 (segment (start 206.1718 77.0382) (end 203.581 74.4728) (width 1) (layer F.Cu) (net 4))
 (segment (start 221.3356 69.8352) (end 220.3852 68.8848) (width 1.2) (layer B.Cu) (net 10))
 (segment (start 221.3356 72.0852) (end 221.3356 69.8352) (width 1.2) (layer B.Cu) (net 10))
 (segment (start 206.121 69.8352) (end 206.121 72.0852) (width 1.2) (layer B.Cu) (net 10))
 (segment (start 207.0714 68.8848) (end 206.121 69.8352) (width 1.2) (layer B.Cu) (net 10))
 (segment (start 220.3852 68.8848) (end 207.0714 68.8848) (width 1.2) (layer B.Cu) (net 10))
 (segment (start 221.361 72.1106) (end 221.3356 72.0852) (width 1) (layer F.Cu) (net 10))
 (segment (start 221.361 78.867) (end 221.361 72.1106) (width 1) (layer F.Cu) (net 10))
 (segment (start 211.455 76.2508) (end 211.455 74.1172) (width 1) (layer F.Cu) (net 9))
 (segment (start 206.5114 85.9104) (end 206.9084 86.3074) (width 0.7) (layer F.Cu) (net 6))
 (via (at 206.9084 87.2998) (size 0.8) (drill 0.4) (layers F.Cu B.Cu) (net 6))
 (segment (start 205.5114 85.9104) (end 206.5114 85.9104) (width 0.7) (layer F.Cu) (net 6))
 (segment (start 206.9084 86.3074) (end 206.9084 87.2998) (width 0.7) (layer F.Cu) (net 6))
 (segment (start 201.168 94.996) (end 206.9084 89.2556) (width 0.7) (layer B.Cu) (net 6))
 (segment (start 201.168 106.2736) (end 201.168 94.996) (width 0.7) (layer B.Cu) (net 6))
 (segment (start 195.072 110.8162) (end 196.6254 110.8162) (width 0.7) (layer B.Cu) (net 6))
 (segment (start 206.9084 89.2556) (end 206.9084 87.2998) (width 0.7) (layer B.Cu) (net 6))
 (segment (start 196.6254 110.8162) (end 201.168 106.2736) (width 0.7) (layer B.Cu) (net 6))
 (segment (start 197.1334 113.3562) (end 195.072 113.3562) (width 0.7) (layer F.Cu) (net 8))
 (segment (start 199.5932 110.8964) (end 197.1334 113.3562) (width 0.7) (layer F.Cu) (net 8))
 (segment (start 199.5932 87.0186) (end 199.5932 110.8964) (width 0.7) (layer F.Cu) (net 8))
 (segment (start 201.7014 85.9104) (end 200.7014 85.9104) (width 0.7) (layer F.Cu) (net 8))
 (segment (start 200.7014 85.9104) (end 199.5932 87.0186) (width 0.7) (layer F.Cu) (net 8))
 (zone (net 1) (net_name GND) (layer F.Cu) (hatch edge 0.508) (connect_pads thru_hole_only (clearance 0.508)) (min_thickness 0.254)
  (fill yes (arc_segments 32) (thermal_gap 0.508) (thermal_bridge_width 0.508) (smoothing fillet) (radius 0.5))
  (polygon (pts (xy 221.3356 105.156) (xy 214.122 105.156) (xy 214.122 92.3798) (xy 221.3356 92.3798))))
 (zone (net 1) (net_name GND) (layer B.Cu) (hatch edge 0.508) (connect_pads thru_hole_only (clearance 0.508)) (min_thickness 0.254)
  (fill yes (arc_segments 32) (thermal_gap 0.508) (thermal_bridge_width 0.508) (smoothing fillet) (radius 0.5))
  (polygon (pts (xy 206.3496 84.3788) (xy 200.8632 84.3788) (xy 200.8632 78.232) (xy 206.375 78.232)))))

